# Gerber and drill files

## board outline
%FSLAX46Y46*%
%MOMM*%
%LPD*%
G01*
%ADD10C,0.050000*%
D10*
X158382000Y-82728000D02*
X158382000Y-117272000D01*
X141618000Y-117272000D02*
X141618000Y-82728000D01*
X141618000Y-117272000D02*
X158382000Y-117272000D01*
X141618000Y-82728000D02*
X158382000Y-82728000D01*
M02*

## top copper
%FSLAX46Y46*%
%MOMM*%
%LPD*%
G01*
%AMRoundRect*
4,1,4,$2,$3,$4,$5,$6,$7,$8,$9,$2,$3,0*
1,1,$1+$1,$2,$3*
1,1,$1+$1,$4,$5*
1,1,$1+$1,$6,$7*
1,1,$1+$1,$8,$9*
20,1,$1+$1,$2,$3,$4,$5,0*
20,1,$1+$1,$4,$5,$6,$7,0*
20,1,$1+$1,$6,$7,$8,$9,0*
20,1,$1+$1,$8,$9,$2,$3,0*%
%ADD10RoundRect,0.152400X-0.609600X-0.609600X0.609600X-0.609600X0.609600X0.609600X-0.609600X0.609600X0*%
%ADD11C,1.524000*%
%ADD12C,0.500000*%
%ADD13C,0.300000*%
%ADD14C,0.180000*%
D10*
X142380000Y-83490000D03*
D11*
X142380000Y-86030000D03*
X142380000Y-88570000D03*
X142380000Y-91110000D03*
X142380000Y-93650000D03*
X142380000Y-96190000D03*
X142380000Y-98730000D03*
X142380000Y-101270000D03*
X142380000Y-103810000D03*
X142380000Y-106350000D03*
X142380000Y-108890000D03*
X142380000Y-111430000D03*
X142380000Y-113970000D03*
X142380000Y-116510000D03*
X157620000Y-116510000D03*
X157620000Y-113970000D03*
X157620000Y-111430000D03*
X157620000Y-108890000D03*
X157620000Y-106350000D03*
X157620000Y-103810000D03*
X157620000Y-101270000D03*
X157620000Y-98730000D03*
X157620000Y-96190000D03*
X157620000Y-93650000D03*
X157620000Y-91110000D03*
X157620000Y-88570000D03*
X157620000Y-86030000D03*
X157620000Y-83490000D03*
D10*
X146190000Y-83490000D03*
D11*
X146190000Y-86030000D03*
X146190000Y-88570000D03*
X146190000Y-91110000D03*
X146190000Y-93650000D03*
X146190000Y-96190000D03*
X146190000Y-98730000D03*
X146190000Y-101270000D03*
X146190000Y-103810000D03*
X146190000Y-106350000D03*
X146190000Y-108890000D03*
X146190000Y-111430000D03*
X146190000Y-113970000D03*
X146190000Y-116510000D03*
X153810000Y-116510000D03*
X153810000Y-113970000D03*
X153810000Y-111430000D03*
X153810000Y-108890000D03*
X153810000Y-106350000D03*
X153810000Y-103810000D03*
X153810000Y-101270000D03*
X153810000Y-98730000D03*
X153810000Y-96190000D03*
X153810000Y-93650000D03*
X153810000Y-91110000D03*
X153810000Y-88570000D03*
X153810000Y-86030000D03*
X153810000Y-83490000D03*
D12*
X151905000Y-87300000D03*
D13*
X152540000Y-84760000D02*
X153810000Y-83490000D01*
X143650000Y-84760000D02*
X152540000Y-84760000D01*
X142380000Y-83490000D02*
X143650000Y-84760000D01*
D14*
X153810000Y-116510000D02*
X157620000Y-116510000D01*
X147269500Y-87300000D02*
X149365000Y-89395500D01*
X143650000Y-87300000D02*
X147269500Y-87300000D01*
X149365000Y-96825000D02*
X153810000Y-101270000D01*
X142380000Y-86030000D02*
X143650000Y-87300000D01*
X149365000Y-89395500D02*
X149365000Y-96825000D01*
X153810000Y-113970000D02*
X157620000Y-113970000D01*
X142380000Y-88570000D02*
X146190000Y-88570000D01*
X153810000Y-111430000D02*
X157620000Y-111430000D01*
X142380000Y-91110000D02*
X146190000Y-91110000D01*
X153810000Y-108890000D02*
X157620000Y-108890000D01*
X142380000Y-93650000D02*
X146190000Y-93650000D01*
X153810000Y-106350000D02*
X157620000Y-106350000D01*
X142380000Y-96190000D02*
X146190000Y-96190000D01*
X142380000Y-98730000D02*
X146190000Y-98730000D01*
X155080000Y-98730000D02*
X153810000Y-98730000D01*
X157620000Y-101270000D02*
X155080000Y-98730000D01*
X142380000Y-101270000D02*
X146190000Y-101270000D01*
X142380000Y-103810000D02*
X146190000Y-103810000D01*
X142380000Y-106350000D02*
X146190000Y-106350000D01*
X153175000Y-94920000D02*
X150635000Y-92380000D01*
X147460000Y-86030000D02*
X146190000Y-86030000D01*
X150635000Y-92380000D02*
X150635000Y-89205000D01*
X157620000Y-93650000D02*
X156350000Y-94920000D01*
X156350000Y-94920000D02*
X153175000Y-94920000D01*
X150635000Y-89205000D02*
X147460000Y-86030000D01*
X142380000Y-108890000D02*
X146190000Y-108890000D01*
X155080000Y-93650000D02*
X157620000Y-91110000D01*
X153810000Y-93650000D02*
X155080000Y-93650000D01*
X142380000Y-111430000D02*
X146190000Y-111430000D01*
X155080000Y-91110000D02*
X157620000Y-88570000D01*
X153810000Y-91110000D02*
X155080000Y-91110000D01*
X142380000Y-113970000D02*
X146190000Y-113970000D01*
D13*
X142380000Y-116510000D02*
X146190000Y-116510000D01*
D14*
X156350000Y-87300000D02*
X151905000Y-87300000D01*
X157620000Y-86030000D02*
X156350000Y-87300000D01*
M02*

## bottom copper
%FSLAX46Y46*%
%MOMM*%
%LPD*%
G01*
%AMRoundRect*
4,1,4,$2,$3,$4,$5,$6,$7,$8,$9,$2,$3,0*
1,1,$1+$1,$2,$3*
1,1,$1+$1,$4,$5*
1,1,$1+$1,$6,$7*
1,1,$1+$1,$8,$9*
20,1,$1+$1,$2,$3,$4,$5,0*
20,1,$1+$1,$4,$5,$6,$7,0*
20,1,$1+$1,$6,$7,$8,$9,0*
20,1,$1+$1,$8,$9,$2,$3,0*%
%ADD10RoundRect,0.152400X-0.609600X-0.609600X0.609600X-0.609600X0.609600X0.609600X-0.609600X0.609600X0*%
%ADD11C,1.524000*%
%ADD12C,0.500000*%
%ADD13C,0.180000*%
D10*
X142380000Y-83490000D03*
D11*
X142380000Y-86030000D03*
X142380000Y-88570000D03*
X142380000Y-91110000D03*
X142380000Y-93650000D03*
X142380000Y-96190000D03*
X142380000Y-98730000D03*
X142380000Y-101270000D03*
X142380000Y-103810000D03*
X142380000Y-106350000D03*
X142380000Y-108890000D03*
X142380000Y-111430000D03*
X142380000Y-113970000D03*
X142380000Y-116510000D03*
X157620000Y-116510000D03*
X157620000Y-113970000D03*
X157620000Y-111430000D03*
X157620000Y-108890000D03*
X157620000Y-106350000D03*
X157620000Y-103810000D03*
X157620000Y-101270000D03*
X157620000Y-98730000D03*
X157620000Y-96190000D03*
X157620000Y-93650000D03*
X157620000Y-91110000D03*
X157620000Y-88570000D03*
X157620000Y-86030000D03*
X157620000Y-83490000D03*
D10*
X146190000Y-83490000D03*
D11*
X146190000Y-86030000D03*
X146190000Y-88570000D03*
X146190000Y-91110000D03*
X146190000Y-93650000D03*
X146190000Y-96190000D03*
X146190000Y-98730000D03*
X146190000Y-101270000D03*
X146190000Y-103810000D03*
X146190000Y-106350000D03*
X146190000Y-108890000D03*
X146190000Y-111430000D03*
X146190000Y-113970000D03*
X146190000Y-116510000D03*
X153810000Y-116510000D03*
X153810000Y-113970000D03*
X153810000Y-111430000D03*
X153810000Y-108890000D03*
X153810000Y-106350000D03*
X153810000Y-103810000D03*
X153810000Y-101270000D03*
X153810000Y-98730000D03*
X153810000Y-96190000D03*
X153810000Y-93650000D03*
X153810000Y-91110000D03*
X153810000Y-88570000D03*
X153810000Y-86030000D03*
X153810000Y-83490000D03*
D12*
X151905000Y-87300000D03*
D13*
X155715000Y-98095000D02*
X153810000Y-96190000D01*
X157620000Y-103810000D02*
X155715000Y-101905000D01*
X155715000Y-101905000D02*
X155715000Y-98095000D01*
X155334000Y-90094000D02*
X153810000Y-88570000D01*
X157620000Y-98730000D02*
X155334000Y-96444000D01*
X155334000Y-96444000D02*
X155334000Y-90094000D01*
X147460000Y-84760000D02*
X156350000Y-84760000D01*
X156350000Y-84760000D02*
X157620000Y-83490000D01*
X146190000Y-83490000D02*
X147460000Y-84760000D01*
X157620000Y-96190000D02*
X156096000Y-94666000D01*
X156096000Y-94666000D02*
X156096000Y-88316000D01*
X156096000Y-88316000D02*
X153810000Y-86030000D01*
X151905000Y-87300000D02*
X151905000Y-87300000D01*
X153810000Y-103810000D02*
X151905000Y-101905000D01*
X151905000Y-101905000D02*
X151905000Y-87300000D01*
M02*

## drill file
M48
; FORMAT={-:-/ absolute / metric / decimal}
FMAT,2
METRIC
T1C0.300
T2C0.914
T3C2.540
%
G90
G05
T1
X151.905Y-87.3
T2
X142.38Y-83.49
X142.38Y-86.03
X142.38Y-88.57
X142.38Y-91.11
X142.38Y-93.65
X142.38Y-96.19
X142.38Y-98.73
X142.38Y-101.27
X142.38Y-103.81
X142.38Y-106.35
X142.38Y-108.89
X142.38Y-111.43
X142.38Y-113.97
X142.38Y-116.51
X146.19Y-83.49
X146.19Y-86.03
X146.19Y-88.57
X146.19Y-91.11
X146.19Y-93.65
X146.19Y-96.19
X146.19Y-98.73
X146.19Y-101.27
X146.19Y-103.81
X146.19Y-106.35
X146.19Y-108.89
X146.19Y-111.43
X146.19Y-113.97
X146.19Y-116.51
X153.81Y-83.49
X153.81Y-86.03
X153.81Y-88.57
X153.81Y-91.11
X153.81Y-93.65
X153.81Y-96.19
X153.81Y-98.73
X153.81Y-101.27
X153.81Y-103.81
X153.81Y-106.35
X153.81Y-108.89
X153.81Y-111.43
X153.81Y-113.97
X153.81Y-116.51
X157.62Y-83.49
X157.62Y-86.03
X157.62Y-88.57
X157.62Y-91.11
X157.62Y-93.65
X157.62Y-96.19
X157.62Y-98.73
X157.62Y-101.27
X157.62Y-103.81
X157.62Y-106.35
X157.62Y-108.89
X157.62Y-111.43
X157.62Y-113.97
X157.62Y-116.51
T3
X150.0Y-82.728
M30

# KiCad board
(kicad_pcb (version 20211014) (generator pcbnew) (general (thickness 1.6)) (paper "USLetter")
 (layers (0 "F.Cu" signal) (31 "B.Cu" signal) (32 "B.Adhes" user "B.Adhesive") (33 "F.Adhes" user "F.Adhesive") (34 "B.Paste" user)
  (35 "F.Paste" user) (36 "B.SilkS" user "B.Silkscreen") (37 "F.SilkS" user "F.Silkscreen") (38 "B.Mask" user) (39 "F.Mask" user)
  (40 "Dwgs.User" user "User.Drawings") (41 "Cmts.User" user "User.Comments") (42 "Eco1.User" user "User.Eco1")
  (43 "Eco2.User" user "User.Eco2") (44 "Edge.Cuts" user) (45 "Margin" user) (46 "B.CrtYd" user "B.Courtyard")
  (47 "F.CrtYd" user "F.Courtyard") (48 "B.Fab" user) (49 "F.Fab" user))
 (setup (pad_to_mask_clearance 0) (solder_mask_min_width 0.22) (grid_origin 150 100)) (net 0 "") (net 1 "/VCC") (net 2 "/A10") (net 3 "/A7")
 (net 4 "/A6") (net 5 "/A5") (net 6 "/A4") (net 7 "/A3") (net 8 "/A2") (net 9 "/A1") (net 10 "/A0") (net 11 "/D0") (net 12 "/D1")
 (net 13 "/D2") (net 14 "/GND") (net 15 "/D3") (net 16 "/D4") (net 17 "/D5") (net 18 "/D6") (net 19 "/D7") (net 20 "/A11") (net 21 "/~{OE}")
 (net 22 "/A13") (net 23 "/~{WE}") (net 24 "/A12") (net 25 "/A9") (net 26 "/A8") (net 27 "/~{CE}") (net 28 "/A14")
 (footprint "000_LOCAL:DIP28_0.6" (layer "F.Cu") (at 150 100)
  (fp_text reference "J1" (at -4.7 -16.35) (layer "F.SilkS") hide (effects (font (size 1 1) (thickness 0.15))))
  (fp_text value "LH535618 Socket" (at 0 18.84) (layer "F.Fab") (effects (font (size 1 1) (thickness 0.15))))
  (pad "1" thru_hole roundrect locked (at -7.62 -16.51) (size 1.524 1.524) (drill 0.9144) (layers *.Cu *.Mask) (roundrect_rratio 0.1)
   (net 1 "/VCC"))
  (pad "2" thru_hole circle locked (at -7.62 -13.97) (size 1.524 1.524) (drill 0.9144) (layers *.Cu *.Mask) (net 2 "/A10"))
  (pad "3" thru_hole circle locked (at -7.62 -11.43) (size 1.524 1.524) (drill 0.9144) (layers *.Cu *.Mask) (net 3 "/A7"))
  (pad "4" thru_hole circle locked (at -7.62 -8.89) (size 1.524 1.524) (drill 0.9144) (layers *.Cu *.Mask) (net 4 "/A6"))
  (pad "5" thru_hole circle locked (at -7.62 -6.35) (size 1.524 1.524) (drill 0.9144) (layers *.Cu *.Mask) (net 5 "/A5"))
  (pad "6" thru_hole circle locked (at -7.62 -3.81) (size 1.524 1.524) (drill 0.9144) (layers *.Cu *.Mask) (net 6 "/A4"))
  (pad "7" thru_hole circle locked (at -7.62 -1.27) (size 1.524 1.524) (drill 0.9144) (layers *.Cu *.Mask) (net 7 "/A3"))
  (pad "8" thru_hole circle locked (at -7.62 1.27) (size 1.524 1.524) (drill 0.9144) (layers *.Cu *.Mask) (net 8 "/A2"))
  (pad "9" thru_hole circle locked (at -7.62 3.81) (size 1.524 1.524) (drill 0.9144) (layers *.Cu *.Mask) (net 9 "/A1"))
  (pad "10" thru_hole circle locked (at -7.62 6.35) (size 1.524 1.524) (drill 0.9144) (layers *.Cu *.Mask) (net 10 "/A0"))
  (pad "11" thru_hole circle locked (at -7.62 8.89) (size 1.524 1.524) (drill 0.9144) (layers *.Cu *.Mask) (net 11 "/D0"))
  (pad "12" thru_hole circle locked (at -7.62 11.43) (size 1.524 1.524) (drill 0.9144) (layers *.Cu *.Mask) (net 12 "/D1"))
  (pad "13" thru_hole circle locked (at -7.62 13.97) (size 1.524 1.524) (drill 0.9144) (layers *.Cu *.Mask) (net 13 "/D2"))
  (pad "14" thru_hole circle locked (at -7.62 16.51) (size 1.524 1.524) (drill 0.9144) (layers *.Cu *.Mask) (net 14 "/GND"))
  (pad "15" thru_hole circle locked (at 7.62 16.51) (size 1.524 1.524) (drill 0.9144) (layers *.Cu *.Mask) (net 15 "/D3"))
  (pad "16" thru_hole circle locked (at 7.62 13.97) (size 1.524 1.524) (drill 0.9144) (layers *.Cu *.Mask) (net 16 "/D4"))
  (pad "17" thru_hole circle locked (at 7.62 11.43) (size 1.524 1.524) (drill 0.9144) (layers *.Cu *.Mask) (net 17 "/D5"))
  (pad "18" thru_hole circle locked (at 7.62 8.89) (size 1.524 1.524) (drill 0.9144) (layers *.Cu *.Mask) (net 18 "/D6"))
  (pad "19" thru_hole circle locked (at 7.62 6.35) (size 1.524 1.524) (drill 0.9144) (layers *.Cu *.Mask) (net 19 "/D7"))
  (pad "20" thru_hole circle locked (at 7.62 3.81) (size 1.524 1.524) (drill 0.9144) (layers *.Cu *.Mask) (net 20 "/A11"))
  (pad "21" thru_hole circle locked (at 7.62 1.27) (size 1.524 1.524) (drill 0.9144) (layers *.Cu *.Mask) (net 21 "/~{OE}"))
  (pad "22" thru_hole circle locked (at 7.62 -1.27) (size 1.524 1.524) (drill 0.9144) (layers *.Cu *.Mask) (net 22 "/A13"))
  (pad "23" thru_hole circle locked (at 7.62 -3.81) (size 1.524 1.524) (drill 0.9144) (layers *.Cu *.Mask) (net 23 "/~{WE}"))
  (pad "24" thru_hole circle locked (at 7.62 -6.35) (size 1.524 1.524) (drill 0.9144) (layers *.Cu *.Mask) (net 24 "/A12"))
  (pad "25" thru_hole circle locked (at 7.62 -8.89) (size 1.524 1.524) (drill 0.9144) (layers *.Cu *.Mask) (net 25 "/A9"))
  (pad "26" thru_hole circle locked (at 7.62 -11.43) (size 1.524 1.524) (drill 0.9144) (layers *.Cu *.Mask) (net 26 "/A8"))
  (pad "27" thru_hole circle locked (at 7.62 -13.97) (size 1.524 1.524) (drill 0.9144) (layers *.Cu *.Mask) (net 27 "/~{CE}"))
  (pad "28" thru_hole circle locked (at 7.62 -16.51) (size 1.524 1.524) (drill 0.9144) (layers *.Cu *.Mask) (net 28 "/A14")))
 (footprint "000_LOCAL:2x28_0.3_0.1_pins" (layer "F.Cu") (at 150 100)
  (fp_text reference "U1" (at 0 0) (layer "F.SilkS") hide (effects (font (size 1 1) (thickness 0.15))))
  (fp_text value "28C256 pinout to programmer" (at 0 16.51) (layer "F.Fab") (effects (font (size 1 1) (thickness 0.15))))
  (pad "1" thru_hole roundrect locked (at -3.81 -16.51) (size 1.524 1.524) (drill 0.9144) (layers *.Cu *.Mask) (roundrect_rratio 0.1)
   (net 28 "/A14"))
  (pad "2" thru_hole circle locked (at -3.81 -13.97) (size 1.524 1.524) (drill 0.9144) (layers *.Cu *.Mask) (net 24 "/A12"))
  (pad "3" thru_hole circle locked (at -3.81 -11.43) (size 1.524 1.524) (drill 0.9144) (layers *.Cu *.Mask) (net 3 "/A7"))
  (pad "4" thru_hole circle locked (at -3.81 -8.89) (size 1.524 1.524) (drill 0.9144) (layers *.Cu *.Mask) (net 4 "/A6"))
  (pad "5" thru_hole circle locked (at -3.81 -6.35) (size 1.524 1.524) (drill 0.9144) (layers *.Cu *.Mask) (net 5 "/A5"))
  (pad "6" thru_hole circle locked (at -3.81 -3.81) (size 1.524 1.524) (drill 0.9144) (layers *.Cu *.Mask) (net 6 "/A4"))
  (pad "7" thru_hole circle locked (at -3.81 -1.27) (size 1.524 1.524) (drill 0.9144) (layers *.Cu *.Mask) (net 7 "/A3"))
  (pad "8" thru_hole circle locked (at -3.81 1.27) (size 1.524 1.524) (drill 0.9144) (layers *.Cu *.Mask) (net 8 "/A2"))
  (pad "9" thru_hole circle locked (at -3.81 3.81) (size 1.524 1.524) (drill 0.9144) (layers *.Cu *.Mask) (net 9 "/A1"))
  (pad "10" thru_hole circle locked (at -3.81 6.35) (size 1.524 1.524) (drill 0.9144) (layers *.Cu *.Mask) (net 10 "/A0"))
  (pad "11" thru_hole circle locked (at -3.81 8.89) (size 1.524 1.524) (drill 0.9144) (layers *.Cu *.Mask) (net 11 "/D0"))
  (pad "12" thru_hole circle locked (at -3.81 11.43) (size 1.524 1.524) (drill 0.9144) (layers *.Cu *.Mask) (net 12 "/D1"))
  (pad "13" thru_hole circle locked (at -3.81 13.97) (size 1.524 1.524) (drill 0.9144) (layers *.Cu *.Mask) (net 13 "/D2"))
  (pad "14" thru_hole circle locked (at -3.81 16.51) (size 1.524 1.524) (drill 0.9144) (layers *.Cu *.Mask) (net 14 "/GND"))
  (pad "15" thru_hole circle locked (at 3.81 16.51) (size 1.524 1.524) (drill 0.9144) (layers *.Cu *.Mask) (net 15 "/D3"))
  (pad "16" thru_hole circle locked (at 3.81 13.97) (size 1.524 1.524) (drill 0.9144) (layers *.Cu *.Mask) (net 16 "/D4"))
  (pad "17" thru_hole circle locked (at 3.81 11.43) (size 1.524 1.524) (drill 0.9144) (layers *.Cu *.Mask) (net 17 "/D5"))
  (pad "18" thru_hole circle locked (at 3.81 8.89) (size 1.524 1.524) (drill 0.9144) (layers *.Cu *.Mask) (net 18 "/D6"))
  (pad "19" thru_hole circle locked (at 3.81 6.35) (size 1.524 1.524) (drill 0.9144) (layers *.Cu *.Mask) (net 19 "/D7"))
  (pad "20" thru_hole circle locked (at 3.81 3.81) (size 1.524 1.524) (drill 0.9144) (layers *.Cu *.Mask) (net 27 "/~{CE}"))
  (pad "21" thru_hole circle locked (at 3.81 1.27) (size 1.524 1.524) (drill 0.9144) (layers *.Cu *.Mask) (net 2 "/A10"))
  (pad "22" thru_hole circle locked (at 3.81 -1.27) (size 1.524 1.524) (drill 0.9144) (layers *.Cu *.Mask) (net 21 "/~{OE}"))
  (pad "23" thru_hole circle locked (at 3.81 -3.81) (size 1.524 1.524) (drill 0.9144) (layers *.Cu *.Mask) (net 20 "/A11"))
  (pad "24" thru_hole circle locked (at 3.81 -6.35) (size 1.524 1.524) (drill 0.9144) (layers *.Cu *.Mask) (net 25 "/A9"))
  (pad "25" thru_hole circle locked (at 3.81 -8.89) (size 1.524 1.524) (drill 0.9144) (layers *.Cu *.Mask) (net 26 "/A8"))
  (pad "26" thru_hole circle locked (at 3.81 -11.43) (size 1.524 1.524) (drill 0.9144) (layers *.Cu *.Mask) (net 22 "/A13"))
  (pad "27" thru_hole circle locked (at 3.81 -13.97) (size 1.524 1.524) (drill 0.9144) (layers *.Cu *.Mask) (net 23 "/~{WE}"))
  (pad "28" thru_hole circle locked (at 3.81 -16.51) (size 1.524 1.524) (drill 0.9144) (layers *.Cu *.Mask) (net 1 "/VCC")))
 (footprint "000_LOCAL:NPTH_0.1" (layer "F.Cu") (at 150 82.728)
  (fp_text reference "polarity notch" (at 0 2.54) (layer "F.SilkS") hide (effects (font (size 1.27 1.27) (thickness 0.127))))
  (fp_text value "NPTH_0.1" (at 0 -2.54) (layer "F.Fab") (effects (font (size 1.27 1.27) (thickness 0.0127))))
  (pad "" np_thru_hole circle locked (at 0 0) (size 2.54 2.54) (drill 2.54) (layers *.Cu *.Mask)))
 (gr_line (start 158.382 82.728) (end 158.382 117.272) (layer "Edge.Cuts") (width 0.05))
 (gr_line (start 141.618 117.272) (end 141.618 82.728) (layer "Edge.Cuts") (width 0.05))
 (gr_line (start 141.618 117.272) (end 158.382 117.272) (layer "Edge.Cuts") (width 0.05))
 (gr_line (start 141.618 82.728) (end 158.382 82.728) (layer "Edge.Cuts") (width 0.05))
 (segment (start 152.54 84.76) (end 153.81 83.49) (width 0.3) (layer "F.Cu") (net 1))
 (segment (start 143.65 84.76) (end 152.54 84.76) (width 0.3) (layer "F.Cu") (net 1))
 (segment (start 142.38 83.49) (end 143.65 84.76) (width 0.3) (layer "F.Cu") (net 1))
 (segment (start 153.81 116.51) (end 157.62 116.51) (width 0.18) (layer "F.Cu") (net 15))
 (segment (start 147.2695 87.3) (end 149.365 89.3955) (width 0.18) (layer "F.Cu") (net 2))
 (segment (start 143.65 87.3) (end 147.2695 87.3) (width 0.18) (layer "F.Cu") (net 2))
 (segment (start 149.365 96.825) (end 153.81 101.27) (width 0.18) (layer "F.Cu") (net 2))
 (segment (start 142.38 86.03) (end 143.65 87.3) (width 0.18) (layer "F.Cu") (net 2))
 (segment (start 149.365 89.3955) (end 149.365 96.825) (width 0.18) (layer "F.Cu") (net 2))
 (segment (start 153.81 113.97) (end 157.62 113.97) (width 0.18) (layer "F.Cu") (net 16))
 (segment (start 142.38 88.57) (end 146.19 88.57) (width 0.18) (layer "F.Cu") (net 3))
 (segment (start 153.81 111.43) (end 157.62 111.43) (width 0.18) (layer "F.Cu") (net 17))
 (segment (start 142.38 91.11) (end 146.19 91.11) (width 0.18) (layer "F.Cu") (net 4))
 (segment (start 153.81 108.89) (end 157.62 108.89) (width 0.18) (layer "F.Cu") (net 18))
 (segment (start 142.38 93.65) (end 146.19 93.65) (width 0.18) (layer "F.Cu") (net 5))
 (segment (start 153.81 106.35) (end 157.62 106.35) (width 0.18) (layer "F.Cu") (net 19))
 (segment (start 142.38 96.19) (end 146.19 96.19) (width 0.18) (layer "F.Cu") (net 6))
 (segment (start 155.715 98.095) (end 153.81 96.19) (width 0.18) (layer "B.Cu") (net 20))
 (segment (start 157.62 103.81) (end 155.715 101.905) (width 0.18) (layer "B.Cu") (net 20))
 (segment (start 155.715 101.905) (end 155.715 98.095) (width 0.18) (layer "B.Cu") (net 20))
 (segment (start 142.38 98.73) (end 146.19 98.73) (width 0.18) (layer "F.Cu") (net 7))
 (segment (start 155.08 98.73) (end 153.81 98.73) (width 0.18) (layer "F.Cu") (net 21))
 (segment (start 157.62 101.27) (end 155.08 98.73) (width 0.18) (layer "F.Cu") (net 21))
 (segment (start 142.38 101.27) (end 146.19 101.27) (width 0.18) (layer "F.Cu") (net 8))
 (segment (start 155.334 90.094) (end 153.81 88.57) (width 0.18) (layer "B.Cu") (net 22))
 (segment (start 157.62 98.73) (end 155.334 96.444) (width 0.18) (layer "B.Cu") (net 22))
 (segment (start 155.334 96.444) (end 155.334 90.094) (width 0.18) (layer "B.Cu") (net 22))
 (segment (start 142.38 103.81) (end 146.19 103.81) (width 0.18) (layer "F.Cu") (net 9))
 (segment (start 142.38 106.35) (end 146.19 106.35) (width 0.18) (layer "F.Cu") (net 10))
 (segment (start 153.175 94.92) (end 150.635 92.38) (width 0.18) (layer "F.Cu") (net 24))
 (segment (start 147.46 86.03) (end 146.19 86.03) (width 0.18) (layer "F.Cu") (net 24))
 (segment (start 150.635 92.38) (end 150.635 89.205) (width 0.18) (layer "F.Cu") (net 24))
 (segment (start 157.62 93.65) (end 156.35 94.92) (width 0.18) (layer "F.Cu") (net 24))
 (segment (start 156.35 94.92) (end 153.175 94.92) (width 0.18) (layer "F.Cu") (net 24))
 (segment (start 150.635 89.205) (end 147.46 86.03) (width 0.18) (layer "F.Cu") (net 24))
 (segment (start 142.38 108.89) (end 146.19 108.89) (width 0.18) (layer "F.Cu") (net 11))
 (segment (start 155.08 93.65) (end 157.62 91.11) (width 0.18) (layer "F.Cu") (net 25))
 (segment (start 153.81 93.65) (end 155.08 93.65) (width 0.18) (layer "F.Cu") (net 25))
 (segment (start 142.38 111.43) (end 146.19 111.43) (width 0.18) (layer "F.Cu") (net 12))
 (segment (start 155.08 91.11) (end 157.62 88.57) (width 0.18) (layer "F.Cu") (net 26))
 (segment (start 153.81 91.11) (end 155.08 91.11) (width 0.18) (layer "F.Cu") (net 26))
 (segment (start 142.38 113.97) (end 146.19 113.97) (width 0.18) (layer "F.Cu") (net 13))
 (segment (start 142.38 116.51) (end 146.19 116.51) (width 0.3) (layer "F.Cu") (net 14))
 (segment (start 147.46 84.76) (end 156.35 84.76) (width 0.18) (layer "B.Cu") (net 28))
 (segment (start 156.35 84.76) (end 157.62 83.49) (width 0.18) (layer "B.Cu") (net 28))
 (segment (start 146.19 83.49) (end 147.46 84.76) (width 0.18) (layer "B.Cu") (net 28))
 (segment (start 157.62 96.19) (end 156.096 94.666) (width 0.18) (layer "B.Cu") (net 23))
 (segment (start 156.096 94.666) (end 156.096 88.316) (width 0.18) (layer "B.Cu") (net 23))
 (segment (start 156.096 88.316) (end 153.81 86.03) (width 0.18) (layer "B.Cu") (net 23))
 (segment (start 156.35 87.3) (end 151.905 87.3) (width 0.18) (layer "F.Cu") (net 27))
 (segment (start 157.62 86.03) (end 156.35 87.3) (width 0.18) (layer "F.Cu") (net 27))
 (via (at 151.905 87.3) (size 0.5) (drill 0.3) (layers "F.Cu" "B.Cu") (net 27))
 (segment (start 151.905 87.3) (end 151.905 87.3) (width 0.18) (layer "B.Cu") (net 27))
 (segment (start 153.81 103.81) (end 151.905 101.905) (width 0.18) (layer "B.Cu") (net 27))
 (segment (start 151.905 101.905) (end 151.905 87.3) (width 0.18) (layer "B.Cu") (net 27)))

